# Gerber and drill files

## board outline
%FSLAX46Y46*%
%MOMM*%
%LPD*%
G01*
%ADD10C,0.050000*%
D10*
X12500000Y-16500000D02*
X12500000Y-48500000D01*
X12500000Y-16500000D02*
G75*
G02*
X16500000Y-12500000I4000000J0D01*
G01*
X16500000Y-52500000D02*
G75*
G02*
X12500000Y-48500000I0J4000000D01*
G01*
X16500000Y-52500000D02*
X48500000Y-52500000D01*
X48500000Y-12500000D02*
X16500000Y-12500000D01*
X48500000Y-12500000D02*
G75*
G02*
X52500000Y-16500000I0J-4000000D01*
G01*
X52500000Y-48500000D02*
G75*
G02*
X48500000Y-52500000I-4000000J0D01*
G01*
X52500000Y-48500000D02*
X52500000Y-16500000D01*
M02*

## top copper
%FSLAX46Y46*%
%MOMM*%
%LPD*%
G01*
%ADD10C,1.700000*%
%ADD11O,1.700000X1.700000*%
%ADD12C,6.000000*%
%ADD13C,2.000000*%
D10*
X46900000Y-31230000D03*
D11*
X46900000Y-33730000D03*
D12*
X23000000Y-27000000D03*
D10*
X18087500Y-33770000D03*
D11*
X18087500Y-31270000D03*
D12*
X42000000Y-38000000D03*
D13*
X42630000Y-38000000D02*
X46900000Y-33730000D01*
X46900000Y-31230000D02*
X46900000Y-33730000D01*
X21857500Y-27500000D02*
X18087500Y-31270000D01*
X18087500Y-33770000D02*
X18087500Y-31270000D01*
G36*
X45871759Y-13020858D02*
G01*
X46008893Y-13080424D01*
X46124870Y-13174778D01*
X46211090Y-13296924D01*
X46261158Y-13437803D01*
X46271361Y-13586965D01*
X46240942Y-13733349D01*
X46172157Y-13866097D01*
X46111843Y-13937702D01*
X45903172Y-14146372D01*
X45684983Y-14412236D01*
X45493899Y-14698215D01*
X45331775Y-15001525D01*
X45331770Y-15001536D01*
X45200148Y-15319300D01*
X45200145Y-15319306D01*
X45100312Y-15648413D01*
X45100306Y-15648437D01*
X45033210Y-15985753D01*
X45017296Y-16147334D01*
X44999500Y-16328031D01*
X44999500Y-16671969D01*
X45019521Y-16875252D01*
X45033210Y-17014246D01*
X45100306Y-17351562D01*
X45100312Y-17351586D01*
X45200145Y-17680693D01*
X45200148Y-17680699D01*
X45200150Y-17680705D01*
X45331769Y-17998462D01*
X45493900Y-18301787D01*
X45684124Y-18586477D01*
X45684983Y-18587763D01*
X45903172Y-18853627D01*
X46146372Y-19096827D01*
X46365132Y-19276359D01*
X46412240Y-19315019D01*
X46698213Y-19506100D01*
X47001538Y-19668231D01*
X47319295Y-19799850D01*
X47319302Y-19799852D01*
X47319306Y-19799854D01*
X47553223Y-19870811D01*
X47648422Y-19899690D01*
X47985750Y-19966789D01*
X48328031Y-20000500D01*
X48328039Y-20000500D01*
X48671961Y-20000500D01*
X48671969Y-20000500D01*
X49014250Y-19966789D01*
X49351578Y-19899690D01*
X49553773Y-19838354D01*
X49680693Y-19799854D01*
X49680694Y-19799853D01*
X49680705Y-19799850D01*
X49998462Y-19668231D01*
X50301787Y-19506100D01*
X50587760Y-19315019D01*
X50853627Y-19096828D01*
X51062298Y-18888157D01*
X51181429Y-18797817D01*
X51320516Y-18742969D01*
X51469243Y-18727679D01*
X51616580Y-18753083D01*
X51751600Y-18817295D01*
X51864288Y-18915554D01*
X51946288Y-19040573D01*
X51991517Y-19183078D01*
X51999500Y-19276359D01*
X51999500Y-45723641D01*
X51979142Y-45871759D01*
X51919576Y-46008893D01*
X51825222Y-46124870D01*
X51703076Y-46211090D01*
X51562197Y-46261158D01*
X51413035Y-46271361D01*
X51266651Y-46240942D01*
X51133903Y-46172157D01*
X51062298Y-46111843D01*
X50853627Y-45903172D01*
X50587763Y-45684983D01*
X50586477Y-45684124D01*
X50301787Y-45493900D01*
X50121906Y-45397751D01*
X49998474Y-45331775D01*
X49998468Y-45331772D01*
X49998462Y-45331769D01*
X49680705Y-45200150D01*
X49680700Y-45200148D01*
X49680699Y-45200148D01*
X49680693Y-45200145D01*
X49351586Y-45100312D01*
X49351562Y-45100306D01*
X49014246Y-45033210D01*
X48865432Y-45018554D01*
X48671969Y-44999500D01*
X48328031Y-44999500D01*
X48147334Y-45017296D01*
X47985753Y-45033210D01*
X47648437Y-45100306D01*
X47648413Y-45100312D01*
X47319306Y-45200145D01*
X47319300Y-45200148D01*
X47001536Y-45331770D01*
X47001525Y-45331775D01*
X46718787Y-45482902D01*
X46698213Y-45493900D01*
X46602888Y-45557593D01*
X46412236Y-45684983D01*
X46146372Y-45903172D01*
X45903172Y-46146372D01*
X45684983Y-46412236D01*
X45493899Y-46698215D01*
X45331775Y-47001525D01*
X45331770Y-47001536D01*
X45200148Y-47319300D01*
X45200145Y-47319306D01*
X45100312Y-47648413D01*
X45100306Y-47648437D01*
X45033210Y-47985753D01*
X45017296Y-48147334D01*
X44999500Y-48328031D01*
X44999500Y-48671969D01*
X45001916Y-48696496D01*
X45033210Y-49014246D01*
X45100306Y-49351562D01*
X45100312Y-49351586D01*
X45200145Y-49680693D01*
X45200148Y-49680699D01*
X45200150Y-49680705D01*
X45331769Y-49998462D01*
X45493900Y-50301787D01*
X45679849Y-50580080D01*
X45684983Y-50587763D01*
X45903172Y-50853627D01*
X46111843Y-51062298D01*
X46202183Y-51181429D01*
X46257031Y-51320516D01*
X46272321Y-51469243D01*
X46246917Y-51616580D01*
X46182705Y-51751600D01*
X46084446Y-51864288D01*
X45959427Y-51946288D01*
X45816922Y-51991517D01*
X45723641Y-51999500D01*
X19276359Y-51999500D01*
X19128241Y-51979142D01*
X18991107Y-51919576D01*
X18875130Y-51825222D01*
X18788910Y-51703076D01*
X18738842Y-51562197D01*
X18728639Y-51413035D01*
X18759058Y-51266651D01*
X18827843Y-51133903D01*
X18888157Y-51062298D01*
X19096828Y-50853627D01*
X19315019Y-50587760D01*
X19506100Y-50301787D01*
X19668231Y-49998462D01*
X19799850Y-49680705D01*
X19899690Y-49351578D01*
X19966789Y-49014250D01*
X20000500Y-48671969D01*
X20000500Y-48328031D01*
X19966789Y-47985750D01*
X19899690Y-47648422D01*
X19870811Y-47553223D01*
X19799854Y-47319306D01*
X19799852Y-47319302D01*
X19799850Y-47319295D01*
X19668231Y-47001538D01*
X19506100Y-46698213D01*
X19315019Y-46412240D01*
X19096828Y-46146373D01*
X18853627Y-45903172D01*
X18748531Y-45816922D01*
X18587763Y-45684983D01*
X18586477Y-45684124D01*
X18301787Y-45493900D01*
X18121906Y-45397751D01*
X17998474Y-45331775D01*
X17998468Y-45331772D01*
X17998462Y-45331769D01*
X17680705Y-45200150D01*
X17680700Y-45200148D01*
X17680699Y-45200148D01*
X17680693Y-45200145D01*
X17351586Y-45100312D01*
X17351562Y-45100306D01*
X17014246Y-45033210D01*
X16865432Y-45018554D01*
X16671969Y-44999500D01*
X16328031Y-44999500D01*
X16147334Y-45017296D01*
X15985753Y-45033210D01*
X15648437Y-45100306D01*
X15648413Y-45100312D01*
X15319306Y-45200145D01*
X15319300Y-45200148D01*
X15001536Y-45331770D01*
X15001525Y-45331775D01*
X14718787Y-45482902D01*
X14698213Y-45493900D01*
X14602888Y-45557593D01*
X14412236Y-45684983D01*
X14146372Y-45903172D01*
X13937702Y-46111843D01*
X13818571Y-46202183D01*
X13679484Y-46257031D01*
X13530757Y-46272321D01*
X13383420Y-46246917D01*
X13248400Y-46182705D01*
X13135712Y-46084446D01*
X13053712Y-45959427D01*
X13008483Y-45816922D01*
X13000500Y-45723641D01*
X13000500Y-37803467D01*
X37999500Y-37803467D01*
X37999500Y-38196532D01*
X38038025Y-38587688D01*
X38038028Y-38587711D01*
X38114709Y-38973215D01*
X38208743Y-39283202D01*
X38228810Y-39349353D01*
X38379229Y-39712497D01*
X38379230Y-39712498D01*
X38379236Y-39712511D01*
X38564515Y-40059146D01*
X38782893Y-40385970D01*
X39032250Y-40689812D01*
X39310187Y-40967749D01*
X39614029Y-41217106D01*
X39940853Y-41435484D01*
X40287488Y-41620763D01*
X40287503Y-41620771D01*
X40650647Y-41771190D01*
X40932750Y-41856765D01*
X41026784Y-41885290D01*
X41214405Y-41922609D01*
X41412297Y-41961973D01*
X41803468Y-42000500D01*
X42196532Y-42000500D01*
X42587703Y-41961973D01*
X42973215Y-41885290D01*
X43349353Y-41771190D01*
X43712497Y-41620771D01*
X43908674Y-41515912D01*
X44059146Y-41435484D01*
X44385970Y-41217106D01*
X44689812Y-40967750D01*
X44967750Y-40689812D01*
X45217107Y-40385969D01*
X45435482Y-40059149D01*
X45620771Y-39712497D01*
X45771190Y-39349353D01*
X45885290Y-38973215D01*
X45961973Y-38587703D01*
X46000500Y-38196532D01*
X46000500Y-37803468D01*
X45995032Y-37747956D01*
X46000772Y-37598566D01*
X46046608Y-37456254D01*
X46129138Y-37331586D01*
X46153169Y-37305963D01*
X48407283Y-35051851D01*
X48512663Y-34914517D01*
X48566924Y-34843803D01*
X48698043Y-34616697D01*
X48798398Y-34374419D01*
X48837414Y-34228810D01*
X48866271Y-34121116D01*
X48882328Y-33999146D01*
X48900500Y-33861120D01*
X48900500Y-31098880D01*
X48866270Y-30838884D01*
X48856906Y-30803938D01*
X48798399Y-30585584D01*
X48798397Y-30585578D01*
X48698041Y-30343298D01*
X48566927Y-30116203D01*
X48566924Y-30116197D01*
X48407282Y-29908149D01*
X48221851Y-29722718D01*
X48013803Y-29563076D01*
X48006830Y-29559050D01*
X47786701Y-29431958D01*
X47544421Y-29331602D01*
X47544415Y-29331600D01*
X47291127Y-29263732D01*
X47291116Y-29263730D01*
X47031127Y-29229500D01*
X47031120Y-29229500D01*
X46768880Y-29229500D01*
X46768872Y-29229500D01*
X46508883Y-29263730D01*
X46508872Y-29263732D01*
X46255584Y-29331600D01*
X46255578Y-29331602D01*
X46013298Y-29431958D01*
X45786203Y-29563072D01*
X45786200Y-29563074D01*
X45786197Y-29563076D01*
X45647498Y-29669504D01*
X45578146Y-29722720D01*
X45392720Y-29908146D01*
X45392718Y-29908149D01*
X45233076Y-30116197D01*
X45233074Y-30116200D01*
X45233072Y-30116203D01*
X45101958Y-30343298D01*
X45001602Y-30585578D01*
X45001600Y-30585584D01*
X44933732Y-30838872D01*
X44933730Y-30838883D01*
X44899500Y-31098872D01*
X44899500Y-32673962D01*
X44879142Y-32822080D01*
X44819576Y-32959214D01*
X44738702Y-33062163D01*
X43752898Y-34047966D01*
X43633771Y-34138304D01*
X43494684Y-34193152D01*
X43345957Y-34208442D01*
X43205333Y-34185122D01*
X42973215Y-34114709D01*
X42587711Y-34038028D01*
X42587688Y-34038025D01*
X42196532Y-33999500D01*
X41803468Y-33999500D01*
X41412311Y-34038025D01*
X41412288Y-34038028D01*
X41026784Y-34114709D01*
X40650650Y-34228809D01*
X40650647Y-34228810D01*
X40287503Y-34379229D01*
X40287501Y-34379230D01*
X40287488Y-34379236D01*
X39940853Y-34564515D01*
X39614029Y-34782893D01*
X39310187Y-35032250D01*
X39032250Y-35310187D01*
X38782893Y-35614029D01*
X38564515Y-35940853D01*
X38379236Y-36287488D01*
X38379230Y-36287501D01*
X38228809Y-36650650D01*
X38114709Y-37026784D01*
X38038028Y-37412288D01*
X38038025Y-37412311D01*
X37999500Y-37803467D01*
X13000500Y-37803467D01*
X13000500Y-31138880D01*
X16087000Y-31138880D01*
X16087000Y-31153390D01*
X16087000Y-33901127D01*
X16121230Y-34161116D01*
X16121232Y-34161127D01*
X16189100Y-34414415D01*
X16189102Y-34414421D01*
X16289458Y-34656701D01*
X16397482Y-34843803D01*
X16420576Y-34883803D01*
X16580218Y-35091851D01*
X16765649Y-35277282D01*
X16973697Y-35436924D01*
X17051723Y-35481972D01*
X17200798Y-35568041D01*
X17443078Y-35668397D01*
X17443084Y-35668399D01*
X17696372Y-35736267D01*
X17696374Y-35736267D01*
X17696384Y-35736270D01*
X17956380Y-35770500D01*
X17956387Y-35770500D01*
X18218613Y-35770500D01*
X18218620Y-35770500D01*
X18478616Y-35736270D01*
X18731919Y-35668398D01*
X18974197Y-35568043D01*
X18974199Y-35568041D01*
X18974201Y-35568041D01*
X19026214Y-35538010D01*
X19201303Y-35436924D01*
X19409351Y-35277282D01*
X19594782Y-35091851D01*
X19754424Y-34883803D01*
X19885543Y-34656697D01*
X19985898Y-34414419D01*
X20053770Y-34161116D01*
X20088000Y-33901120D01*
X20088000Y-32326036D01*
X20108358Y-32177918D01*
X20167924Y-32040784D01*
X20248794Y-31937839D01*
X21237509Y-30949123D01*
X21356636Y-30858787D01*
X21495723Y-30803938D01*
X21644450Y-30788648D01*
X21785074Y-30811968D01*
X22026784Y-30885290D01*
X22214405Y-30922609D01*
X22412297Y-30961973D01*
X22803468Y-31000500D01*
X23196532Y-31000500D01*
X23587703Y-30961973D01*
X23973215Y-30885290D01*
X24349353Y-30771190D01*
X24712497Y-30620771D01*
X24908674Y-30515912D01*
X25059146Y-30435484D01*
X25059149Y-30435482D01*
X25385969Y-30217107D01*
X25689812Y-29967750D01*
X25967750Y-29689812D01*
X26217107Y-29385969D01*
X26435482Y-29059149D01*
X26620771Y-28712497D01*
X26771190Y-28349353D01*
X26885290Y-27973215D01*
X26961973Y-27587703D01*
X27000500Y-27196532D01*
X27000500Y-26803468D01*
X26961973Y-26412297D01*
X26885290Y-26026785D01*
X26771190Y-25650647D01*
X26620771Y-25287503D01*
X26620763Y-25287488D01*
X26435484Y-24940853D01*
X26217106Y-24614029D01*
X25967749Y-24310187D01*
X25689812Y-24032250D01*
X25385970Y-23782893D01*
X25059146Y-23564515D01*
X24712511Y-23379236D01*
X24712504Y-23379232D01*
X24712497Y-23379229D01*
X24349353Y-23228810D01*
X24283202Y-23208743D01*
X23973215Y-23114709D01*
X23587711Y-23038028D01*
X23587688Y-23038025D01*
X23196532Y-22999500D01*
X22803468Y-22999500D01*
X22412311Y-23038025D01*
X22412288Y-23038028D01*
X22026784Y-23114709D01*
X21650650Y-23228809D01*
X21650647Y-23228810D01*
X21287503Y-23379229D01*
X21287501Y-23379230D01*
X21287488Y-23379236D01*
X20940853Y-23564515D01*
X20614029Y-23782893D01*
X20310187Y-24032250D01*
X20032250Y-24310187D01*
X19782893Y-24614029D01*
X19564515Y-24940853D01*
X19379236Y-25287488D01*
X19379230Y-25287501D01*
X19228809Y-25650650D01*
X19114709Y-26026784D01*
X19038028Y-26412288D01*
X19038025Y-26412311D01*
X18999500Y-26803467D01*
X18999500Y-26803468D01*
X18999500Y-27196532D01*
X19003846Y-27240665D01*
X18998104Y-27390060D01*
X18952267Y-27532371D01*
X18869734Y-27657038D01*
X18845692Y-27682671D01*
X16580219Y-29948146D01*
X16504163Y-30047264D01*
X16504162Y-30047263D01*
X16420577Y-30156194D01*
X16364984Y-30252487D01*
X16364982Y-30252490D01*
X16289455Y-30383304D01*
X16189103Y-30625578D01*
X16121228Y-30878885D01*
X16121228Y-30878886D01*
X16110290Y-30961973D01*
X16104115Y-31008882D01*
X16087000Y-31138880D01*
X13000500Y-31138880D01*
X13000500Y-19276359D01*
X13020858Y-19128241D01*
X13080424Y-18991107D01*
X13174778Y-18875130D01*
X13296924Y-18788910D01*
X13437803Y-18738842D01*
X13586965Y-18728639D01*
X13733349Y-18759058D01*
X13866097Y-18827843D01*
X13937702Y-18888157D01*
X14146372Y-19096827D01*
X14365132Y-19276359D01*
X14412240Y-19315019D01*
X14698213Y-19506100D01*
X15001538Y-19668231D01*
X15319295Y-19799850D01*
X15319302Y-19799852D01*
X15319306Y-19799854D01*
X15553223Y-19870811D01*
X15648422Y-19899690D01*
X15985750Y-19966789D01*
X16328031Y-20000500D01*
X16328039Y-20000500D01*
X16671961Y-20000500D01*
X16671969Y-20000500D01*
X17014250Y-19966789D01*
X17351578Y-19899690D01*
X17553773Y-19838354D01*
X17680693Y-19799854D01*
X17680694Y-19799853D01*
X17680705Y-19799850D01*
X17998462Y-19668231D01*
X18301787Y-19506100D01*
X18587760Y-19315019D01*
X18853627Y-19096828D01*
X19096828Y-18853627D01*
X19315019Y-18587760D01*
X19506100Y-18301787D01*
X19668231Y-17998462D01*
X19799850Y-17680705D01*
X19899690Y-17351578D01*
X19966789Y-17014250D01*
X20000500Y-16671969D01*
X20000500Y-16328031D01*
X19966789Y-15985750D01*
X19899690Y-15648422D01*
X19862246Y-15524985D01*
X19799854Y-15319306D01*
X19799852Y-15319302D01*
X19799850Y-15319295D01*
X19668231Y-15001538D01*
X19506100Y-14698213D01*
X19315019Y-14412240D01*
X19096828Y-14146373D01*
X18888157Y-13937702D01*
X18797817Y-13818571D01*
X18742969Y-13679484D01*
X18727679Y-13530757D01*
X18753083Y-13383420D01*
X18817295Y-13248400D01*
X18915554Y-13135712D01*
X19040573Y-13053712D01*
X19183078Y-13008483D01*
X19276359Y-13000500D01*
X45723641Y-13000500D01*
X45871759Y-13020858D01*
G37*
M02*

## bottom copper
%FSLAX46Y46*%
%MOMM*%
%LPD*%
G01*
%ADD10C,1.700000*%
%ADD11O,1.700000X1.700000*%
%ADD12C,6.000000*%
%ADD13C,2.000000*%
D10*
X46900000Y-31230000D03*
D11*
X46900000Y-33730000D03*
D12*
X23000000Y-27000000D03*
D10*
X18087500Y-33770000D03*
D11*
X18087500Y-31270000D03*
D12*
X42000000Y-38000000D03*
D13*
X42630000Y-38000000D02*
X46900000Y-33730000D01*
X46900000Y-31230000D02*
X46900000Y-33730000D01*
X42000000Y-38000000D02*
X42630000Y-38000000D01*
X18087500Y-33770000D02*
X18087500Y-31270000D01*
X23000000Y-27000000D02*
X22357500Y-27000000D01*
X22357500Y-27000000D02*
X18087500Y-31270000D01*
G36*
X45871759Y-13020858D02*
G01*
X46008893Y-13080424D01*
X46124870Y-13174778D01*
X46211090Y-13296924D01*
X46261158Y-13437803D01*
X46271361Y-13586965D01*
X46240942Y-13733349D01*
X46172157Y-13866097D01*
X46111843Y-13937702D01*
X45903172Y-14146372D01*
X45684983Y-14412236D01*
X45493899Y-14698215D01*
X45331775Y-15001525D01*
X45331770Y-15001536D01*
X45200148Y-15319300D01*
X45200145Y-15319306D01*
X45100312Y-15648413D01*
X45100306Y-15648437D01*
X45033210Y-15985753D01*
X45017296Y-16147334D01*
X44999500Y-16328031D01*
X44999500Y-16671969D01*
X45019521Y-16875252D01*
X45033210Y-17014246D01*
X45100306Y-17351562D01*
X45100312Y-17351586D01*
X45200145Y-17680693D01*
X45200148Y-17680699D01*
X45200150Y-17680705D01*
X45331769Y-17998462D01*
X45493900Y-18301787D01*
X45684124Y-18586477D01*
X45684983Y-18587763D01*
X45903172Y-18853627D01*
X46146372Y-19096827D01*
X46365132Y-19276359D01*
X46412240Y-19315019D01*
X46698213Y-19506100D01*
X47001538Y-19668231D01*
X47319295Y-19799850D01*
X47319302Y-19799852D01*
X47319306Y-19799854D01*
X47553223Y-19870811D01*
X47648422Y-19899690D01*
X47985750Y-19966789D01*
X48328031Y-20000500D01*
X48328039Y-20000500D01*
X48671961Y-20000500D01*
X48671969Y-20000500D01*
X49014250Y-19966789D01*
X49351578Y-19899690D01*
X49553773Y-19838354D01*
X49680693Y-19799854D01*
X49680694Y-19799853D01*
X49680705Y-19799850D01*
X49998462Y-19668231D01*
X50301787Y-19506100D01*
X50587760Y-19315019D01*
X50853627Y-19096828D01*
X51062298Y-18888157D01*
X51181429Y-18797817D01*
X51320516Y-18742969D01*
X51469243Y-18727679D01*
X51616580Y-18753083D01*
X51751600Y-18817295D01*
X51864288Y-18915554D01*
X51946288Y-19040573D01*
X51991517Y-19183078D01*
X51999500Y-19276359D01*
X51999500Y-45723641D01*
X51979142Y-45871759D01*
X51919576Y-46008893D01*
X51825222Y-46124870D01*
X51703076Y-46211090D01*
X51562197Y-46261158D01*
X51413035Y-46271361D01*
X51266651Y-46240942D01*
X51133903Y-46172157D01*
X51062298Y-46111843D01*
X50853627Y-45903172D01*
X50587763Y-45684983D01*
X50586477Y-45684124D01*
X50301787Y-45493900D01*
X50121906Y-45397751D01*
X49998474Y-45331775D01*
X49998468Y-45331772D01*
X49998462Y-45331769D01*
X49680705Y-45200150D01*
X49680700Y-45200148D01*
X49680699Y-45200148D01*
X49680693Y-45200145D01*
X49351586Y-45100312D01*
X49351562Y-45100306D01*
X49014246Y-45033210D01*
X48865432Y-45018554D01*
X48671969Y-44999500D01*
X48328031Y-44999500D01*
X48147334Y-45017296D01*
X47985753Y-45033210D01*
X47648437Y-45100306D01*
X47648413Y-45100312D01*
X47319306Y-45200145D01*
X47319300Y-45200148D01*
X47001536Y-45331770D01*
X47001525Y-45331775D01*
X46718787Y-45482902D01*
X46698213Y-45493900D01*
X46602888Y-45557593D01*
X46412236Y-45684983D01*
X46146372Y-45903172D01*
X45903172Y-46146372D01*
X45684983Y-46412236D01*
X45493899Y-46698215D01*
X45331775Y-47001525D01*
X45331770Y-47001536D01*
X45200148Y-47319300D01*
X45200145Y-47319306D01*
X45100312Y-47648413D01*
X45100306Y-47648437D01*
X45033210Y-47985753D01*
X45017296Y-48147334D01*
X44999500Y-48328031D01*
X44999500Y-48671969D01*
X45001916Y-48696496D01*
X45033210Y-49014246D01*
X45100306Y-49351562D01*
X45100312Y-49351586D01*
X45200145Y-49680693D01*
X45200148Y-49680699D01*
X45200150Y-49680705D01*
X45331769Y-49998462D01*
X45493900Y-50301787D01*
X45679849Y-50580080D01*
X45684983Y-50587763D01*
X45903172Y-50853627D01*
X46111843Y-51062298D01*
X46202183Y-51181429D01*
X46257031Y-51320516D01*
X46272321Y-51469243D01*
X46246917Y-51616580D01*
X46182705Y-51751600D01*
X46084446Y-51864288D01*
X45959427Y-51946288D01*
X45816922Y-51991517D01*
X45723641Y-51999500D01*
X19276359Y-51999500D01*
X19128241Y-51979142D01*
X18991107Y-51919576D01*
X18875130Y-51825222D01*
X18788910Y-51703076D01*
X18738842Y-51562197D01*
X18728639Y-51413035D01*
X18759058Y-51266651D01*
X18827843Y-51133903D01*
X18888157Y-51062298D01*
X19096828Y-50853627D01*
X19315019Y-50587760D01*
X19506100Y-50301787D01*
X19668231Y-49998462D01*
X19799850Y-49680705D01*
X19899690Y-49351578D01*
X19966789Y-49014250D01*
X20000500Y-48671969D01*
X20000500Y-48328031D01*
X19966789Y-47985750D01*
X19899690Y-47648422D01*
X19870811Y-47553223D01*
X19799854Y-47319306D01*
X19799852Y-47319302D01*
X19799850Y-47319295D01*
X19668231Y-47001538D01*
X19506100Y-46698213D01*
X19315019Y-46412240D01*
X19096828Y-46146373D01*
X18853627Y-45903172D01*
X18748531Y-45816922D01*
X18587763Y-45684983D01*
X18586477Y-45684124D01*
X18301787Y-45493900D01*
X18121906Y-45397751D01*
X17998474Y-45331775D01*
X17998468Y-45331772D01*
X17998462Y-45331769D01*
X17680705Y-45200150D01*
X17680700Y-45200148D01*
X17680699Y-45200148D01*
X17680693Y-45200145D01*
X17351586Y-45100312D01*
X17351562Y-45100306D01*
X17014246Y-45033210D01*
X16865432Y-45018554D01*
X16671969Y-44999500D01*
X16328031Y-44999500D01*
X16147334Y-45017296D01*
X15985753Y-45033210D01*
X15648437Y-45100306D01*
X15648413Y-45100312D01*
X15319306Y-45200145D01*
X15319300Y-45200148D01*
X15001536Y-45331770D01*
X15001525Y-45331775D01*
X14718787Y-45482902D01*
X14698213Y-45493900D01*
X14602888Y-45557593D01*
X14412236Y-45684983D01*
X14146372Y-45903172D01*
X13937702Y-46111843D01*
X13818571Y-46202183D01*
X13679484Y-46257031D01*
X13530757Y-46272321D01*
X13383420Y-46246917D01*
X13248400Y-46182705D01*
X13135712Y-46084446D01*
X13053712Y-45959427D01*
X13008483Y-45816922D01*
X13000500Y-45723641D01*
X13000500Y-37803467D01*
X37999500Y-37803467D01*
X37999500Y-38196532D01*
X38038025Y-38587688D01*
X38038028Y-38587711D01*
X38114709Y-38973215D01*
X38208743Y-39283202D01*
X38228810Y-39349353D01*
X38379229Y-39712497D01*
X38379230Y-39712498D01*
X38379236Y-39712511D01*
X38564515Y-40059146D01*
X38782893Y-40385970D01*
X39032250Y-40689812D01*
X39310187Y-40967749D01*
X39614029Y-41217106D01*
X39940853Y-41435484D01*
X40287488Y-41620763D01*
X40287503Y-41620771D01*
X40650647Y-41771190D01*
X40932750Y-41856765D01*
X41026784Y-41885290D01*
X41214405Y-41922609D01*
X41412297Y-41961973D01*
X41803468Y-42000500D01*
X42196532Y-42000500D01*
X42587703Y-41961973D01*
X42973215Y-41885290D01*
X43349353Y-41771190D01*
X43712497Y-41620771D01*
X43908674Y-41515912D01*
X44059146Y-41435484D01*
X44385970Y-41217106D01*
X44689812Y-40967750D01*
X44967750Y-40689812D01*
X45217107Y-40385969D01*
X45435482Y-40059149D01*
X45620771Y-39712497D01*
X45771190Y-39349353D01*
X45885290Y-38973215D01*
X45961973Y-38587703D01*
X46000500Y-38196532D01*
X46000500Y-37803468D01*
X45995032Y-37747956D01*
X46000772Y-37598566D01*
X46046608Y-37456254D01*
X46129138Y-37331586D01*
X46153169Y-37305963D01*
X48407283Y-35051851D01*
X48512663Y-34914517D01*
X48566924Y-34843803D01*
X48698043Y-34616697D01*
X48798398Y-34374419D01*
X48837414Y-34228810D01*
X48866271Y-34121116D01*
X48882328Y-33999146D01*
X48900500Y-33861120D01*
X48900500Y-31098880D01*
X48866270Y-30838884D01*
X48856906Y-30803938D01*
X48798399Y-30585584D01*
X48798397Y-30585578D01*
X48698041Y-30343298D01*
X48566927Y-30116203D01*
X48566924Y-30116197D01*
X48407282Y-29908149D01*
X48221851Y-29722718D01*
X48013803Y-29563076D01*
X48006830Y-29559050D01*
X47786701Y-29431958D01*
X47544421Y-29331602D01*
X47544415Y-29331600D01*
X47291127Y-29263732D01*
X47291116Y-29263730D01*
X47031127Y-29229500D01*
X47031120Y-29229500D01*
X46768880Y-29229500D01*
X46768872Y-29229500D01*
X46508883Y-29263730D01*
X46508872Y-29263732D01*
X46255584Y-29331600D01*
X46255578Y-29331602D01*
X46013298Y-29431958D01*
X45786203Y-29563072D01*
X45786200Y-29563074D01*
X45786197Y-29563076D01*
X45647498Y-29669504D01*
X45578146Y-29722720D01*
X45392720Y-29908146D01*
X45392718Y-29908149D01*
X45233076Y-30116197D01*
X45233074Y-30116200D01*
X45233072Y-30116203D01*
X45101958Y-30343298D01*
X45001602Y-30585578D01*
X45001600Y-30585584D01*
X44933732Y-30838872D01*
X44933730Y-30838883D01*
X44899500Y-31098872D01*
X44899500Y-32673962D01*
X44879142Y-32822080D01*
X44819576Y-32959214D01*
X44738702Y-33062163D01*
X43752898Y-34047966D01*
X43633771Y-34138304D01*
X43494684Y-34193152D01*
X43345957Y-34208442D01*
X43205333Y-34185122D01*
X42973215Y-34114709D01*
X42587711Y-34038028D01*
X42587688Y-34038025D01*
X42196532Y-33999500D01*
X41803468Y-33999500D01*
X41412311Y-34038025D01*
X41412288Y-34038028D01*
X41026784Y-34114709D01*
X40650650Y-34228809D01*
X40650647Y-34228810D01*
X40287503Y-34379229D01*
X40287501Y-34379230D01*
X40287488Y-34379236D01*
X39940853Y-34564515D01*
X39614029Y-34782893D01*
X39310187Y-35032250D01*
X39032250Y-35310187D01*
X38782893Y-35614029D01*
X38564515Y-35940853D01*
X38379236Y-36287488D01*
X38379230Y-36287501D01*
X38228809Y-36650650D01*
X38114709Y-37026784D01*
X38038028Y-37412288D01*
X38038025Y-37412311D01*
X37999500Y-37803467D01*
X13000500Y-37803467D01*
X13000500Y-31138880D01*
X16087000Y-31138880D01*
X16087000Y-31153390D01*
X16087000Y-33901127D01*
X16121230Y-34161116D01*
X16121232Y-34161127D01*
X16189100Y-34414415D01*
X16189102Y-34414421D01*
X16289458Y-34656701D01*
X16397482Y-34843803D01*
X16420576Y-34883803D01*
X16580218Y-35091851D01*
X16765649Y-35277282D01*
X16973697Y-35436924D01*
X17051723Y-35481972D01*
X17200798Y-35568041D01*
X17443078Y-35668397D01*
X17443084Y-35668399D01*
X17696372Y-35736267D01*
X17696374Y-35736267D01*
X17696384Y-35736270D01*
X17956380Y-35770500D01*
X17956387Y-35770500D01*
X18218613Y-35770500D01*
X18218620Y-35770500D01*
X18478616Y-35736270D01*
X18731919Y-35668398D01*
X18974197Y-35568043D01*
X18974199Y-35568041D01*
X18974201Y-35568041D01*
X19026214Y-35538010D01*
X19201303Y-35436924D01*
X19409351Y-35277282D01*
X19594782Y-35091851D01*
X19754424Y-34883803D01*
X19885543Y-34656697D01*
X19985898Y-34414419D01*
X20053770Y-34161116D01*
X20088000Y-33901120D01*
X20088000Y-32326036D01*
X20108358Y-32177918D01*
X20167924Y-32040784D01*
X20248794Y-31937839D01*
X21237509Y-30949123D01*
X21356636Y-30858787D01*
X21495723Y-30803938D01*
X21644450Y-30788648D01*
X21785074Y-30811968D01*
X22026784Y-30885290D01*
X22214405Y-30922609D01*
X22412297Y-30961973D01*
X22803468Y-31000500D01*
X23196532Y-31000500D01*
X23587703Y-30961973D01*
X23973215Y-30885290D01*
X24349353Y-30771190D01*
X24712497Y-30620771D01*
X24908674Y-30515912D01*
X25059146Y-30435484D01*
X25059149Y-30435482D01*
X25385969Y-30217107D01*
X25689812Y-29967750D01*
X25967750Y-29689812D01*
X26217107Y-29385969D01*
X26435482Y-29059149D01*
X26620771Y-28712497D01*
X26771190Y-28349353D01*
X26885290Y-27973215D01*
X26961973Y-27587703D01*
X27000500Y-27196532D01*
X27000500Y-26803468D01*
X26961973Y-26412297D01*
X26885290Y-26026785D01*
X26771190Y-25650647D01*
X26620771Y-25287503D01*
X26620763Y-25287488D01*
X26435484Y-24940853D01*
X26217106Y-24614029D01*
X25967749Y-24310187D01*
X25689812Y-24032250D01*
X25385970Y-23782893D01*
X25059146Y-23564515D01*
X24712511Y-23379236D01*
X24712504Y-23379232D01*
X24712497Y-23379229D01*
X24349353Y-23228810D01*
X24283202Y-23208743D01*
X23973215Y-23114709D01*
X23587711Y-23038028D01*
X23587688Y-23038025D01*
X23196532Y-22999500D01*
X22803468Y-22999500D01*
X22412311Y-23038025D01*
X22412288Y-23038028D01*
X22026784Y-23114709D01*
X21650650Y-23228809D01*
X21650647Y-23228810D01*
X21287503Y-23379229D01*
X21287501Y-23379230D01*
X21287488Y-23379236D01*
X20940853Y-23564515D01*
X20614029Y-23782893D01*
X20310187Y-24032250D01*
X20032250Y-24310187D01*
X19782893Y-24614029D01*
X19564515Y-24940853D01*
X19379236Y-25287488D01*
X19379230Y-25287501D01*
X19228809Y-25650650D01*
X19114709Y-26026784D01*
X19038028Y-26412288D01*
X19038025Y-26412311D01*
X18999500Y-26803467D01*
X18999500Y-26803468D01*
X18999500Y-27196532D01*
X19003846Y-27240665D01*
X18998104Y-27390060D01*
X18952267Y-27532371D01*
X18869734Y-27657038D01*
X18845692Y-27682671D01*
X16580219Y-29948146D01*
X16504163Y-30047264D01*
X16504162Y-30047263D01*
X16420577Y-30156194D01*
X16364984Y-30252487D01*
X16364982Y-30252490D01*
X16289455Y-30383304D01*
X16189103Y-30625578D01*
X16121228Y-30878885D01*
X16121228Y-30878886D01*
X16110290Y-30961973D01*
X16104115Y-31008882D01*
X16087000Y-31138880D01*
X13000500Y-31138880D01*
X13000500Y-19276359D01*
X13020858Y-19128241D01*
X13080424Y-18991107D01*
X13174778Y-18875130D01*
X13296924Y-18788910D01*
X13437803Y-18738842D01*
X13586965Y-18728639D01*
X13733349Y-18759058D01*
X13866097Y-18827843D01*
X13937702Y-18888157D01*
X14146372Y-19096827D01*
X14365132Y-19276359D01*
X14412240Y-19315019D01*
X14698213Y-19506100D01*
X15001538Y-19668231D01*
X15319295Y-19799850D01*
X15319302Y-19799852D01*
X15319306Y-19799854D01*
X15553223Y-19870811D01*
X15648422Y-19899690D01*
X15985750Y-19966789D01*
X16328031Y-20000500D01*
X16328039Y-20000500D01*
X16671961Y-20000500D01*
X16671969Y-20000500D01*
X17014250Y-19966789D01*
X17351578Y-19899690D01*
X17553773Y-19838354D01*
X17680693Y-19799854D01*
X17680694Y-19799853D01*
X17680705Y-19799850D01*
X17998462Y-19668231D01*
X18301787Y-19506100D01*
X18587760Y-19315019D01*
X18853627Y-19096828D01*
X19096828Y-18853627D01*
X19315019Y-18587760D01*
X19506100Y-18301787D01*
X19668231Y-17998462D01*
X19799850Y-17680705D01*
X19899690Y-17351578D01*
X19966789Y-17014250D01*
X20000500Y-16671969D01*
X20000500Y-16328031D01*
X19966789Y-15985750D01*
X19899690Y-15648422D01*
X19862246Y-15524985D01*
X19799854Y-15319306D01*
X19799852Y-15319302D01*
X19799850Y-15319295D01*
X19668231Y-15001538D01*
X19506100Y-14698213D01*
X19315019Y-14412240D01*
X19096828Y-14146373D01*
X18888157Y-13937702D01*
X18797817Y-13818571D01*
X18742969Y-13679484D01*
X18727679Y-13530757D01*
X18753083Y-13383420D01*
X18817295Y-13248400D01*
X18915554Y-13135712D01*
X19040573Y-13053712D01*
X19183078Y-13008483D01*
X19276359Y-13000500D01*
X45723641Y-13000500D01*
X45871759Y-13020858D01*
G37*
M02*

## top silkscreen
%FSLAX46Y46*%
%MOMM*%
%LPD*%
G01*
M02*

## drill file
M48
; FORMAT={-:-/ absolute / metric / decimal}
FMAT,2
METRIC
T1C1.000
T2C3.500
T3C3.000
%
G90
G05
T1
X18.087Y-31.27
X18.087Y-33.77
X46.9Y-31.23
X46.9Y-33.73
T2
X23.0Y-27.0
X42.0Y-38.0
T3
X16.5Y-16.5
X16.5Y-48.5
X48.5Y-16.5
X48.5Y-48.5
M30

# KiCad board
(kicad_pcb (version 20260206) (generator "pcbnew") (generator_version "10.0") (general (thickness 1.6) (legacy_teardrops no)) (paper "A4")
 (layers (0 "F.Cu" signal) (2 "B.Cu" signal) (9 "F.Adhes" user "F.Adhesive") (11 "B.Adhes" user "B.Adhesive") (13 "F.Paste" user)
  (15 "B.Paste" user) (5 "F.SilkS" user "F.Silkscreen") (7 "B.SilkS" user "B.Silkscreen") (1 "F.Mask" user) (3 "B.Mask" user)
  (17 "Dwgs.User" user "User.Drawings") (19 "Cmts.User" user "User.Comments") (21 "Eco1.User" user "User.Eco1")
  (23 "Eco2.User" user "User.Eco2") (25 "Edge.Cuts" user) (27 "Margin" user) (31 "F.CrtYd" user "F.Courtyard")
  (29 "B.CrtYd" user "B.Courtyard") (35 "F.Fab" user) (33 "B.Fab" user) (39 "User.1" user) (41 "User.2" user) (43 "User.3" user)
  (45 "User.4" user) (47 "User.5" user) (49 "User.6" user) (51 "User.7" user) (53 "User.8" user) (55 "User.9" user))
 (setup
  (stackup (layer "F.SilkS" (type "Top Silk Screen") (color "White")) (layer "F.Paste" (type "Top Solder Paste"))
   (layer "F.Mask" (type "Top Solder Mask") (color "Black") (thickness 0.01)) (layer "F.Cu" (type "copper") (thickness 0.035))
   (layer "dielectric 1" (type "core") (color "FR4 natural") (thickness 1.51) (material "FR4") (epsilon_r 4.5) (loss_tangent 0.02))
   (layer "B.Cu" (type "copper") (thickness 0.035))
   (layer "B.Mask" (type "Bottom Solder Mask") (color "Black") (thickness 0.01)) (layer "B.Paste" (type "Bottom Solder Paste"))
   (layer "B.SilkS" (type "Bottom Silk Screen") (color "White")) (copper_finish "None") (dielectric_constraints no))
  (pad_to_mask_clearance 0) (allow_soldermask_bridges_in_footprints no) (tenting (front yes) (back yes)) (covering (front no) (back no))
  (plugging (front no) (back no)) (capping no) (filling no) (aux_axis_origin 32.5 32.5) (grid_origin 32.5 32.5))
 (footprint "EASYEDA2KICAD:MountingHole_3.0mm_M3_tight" (layer "F.Cu") (at 48.5 48.5 -90)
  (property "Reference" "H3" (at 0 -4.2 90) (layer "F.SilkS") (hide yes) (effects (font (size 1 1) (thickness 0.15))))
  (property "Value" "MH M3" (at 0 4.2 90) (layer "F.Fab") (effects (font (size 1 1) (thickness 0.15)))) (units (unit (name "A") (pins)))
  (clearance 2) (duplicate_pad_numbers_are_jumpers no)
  (pad "" np_thru_hole circle (at 0 0 270) (size 3 3) (drill 3) (layers "*.Cu" "*.Mask")))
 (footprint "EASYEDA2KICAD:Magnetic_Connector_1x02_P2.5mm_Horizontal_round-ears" (layer "F.Cu") (at 47 32.5)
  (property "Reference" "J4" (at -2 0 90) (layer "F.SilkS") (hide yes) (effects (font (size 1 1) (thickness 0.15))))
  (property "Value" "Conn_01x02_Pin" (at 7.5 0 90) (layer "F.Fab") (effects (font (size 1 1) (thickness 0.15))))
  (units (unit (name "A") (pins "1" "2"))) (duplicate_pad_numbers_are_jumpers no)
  (pad "1" thru_hole circle (at -0.1 -1.27) (size 1.7 1.7) (drill 1) (layers "*.Cu" "*.Mask") (remove_unused_layers no)
   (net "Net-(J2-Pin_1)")
   (teardrops (best_length_ratio 0.5) (max_length 1) (best_width_ratio 1) (max_width 2) (curved_edges yes) (filter_ratio 0.9) (enabled yes)
    (allow_two_segments yes) (prefer_zone_connections yes)))
  (pad "2" thru_hole oval (at -0.1 1.23) (size 1.7 1.7) (drill 1) (layers "*.Cu" "*.Mask") (remove_unused_layers no) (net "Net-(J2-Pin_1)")
   (teardrops (best_length_ratio 0.5) (max_length 1) (best_width_ratio 1) (max_width 2) (curved_edges yes) (filter_ratio 0.9) (enabled yes)
    (allow_two_segments yes) (prefer_zone_connections yes))))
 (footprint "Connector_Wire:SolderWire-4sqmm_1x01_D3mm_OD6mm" (layer "F.Cu") (at 23 27 -90)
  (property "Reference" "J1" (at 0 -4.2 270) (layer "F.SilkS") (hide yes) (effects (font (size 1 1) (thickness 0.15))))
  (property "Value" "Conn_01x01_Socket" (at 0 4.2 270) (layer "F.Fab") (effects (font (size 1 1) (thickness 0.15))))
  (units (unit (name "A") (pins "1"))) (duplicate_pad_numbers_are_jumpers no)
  (pad "1" thru_hole circle (at 0 0 270) (size 6 6) (drill 3.5) (layers "*.Cu" "*.Mask") (remove_unused_layers no) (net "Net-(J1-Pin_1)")
   (teardrops (best_length_ratio 0.5) (max_length 1) (best_width_ratio 1) (max_width 2) (curved_edges yes) (filter_ratio 0.9) (enabled yes)
    (allow_two_segments yes) (prefer_zone_connections yes))))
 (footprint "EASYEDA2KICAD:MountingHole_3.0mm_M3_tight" (layer "F.Cu") (at 48.5 16.5 -90)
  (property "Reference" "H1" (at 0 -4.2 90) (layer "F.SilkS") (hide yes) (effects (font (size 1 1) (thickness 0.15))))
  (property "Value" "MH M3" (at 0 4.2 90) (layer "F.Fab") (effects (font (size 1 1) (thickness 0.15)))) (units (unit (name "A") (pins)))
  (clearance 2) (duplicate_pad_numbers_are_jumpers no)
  (pad "" np_thru_hole circle (at 0 0 270) (size 3 3) (drill 3) (layers "*.Cu" "*.Mask")))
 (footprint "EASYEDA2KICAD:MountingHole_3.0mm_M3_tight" (layer "F.Cu") (at 16.5 48.5 -90)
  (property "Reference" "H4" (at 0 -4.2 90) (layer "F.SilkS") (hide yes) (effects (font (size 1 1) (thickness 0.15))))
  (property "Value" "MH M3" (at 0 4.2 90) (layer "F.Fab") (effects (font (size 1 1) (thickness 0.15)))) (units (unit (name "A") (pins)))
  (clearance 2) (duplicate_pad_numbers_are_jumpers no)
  (pad "" np_thru_hole circle (at 0 0 270) (size 3 3) (drill 3) (layers "*.Cu" "*.Mask")))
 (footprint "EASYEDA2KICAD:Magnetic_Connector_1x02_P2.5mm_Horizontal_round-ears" (layer "F.Cu") (at 17.9875 32.5 180)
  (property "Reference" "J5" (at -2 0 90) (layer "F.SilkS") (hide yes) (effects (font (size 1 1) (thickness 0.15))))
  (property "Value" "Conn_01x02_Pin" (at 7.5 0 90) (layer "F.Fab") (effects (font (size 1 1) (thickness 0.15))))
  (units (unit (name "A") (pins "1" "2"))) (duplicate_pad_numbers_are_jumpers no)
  (pad "1" thru_hole circle (at -0.1 -1.27 180) (size 1.7 1.7) (drill 1) (layers "*.Cu" "*.Mask") (remove_unused_layers no)
   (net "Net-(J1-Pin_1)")
   (teardrops (best_length_ratio 0.5) (max_length 1) (best_width_ratio 1) (max_width 2) (curved_edges yes) (filter_ratio 0.9) (enabled yes)
    (allow_two_segments yes) (prefer_zone_connections yes)))
  (pad "2" thru_hole oval (at -0.1 1.23 180) (size 1.7 1.7) (drill 1) (layers "*.Cu" "*.Mask") (remove_unused_layers no)
   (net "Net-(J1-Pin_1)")
   (teardrops (best_length_ratio 0.5) (max_length 1) (best_width_ratio 1) (max_width 2) (curved_edges yes) (filter_ratio 0.9) (enabled yes)
    (allow_two_segments yes) (prefer_zone_connections yes))))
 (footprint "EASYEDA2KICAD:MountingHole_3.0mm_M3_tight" (layer "F.Cu") (at 16.5 16.5 -90)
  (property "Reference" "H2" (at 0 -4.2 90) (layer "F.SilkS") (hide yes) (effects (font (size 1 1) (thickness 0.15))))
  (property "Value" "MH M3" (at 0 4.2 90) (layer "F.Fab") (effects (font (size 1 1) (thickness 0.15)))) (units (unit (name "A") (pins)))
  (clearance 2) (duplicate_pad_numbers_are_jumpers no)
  (pad "" np_thru_hole circle (at 0 0 270) (size 3 3) (drill 3) (layers "*.Cu" "*.Mask")))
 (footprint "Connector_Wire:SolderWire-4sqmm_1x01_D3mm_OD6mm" (layer "F.Cu") (at 42 38 -90)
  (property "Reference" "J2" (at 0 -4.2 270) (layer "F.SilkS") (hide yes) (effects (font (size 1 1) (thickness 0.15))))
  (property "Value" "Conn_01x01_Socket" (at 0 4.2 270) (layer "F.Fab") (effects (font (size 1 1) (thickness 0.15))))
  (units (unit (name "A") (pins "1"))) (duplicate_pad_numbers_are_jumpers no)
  (pad "1" thru_hole circle (at 0 0 270) (size 6 6) (drill 3.5) (layers "*.Cu" "*.Mask") (remove_unused_layers no) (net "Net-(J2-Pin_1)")
   (teardrops (best_length_ratio 0.5) (max_length 1) (best_width_ratio 1) (max_width 2) (curved_edges yes) (filter_ratio 0.9) (enabled yes)
    (allow_two_segments yes) (prefer_zone_connections yes))))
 (gr_line (start 12.5 16.5) (end 12.5 48.5) (stroke (width 0.05) (type default)) (layer "Edge.Cuts"))
 (gr_arc (start 12.5 16.5) (mid 13.671573 13.671573) (end 16.5 12.5) (stroke (width 0.05) (type default)) (layer "Edge.Cuts"))
 (gr_arc (start 16.5 52.5) (mid 13.671573 51.328427) (end 12.5 48.5) (stroke (width 0.05) (type default)) (layer "Edge.Cuts"))
 (gr_line (start 16.5 52.5) (end 48.5 52.5) (stroke (width 0.05) (type default)) (layer "Edge.Cuts"))
 (gr_line (start 48.5 12.5) (end 16.5 12.5) (stroke (width 0.05) (type default)) (layer "Edge.Cuts"))
 (gr_arc (start 48.5 12.5) (mid 51.328427 13.671573) (end 52.5 16.5) (stroke (width 0.05) (type default)) (layer "Edge.Cuts"))
 (gr_arc (start 52.5 48.5) (mid 51.328427 51.328427) (end 48.5 52.5) (stroke (width 0.05) (type default)) (layer "Edge.Cuts"))
 (gr_line (start 52.5 48.5) (end 52.5 16.5) (stroke (width 0.05) (type default)) (layer "Edge.Cuts"))
 (segment (start 42.63 38) (end 46.9 33.73) (width 2) (layer "F.Cu") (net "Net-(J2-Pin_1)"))
 (segment (start 46.9 31.23) (end 46.9 33.73) (width 2) (layer "F.Cu") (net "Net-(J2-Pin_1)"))
 (segment (start 42.63 38) (end 46.9 33.73) (width 2) (layer "B.Cu") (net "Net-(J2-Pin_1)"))
 (segment (start 46.9 31.23) (end 46.9 33.73) (width 2) (layer "B.Cu") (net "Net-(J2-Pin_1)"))
 (segment (start 42 38) (end 42.63 38) (width 2) (layer "B.Cu") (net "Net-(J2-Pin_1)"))
 (segment (start 21.8575 27.5) (end 18.0875 31.27) (width 2) (layer "F.Cu") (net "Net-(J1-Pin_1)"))
 (segment (start 18.0875 33.77) (end 18.0875 31.27) (width 2) (layer "F.Cu") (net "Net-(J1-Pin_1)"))
 (segment (start 18.0875 33.77) (end 18.0875 31.27) (width 2) (layer "B.Cu") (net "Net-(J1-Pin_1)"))
 (segment (start 23 27) (end 22.3575 27) (width 2) (layer "B.Cu") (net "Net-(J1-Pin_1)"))
 (segment (start 22.3575 27) (end 18.0875 31.27) (width 2) (layer "B.Cu") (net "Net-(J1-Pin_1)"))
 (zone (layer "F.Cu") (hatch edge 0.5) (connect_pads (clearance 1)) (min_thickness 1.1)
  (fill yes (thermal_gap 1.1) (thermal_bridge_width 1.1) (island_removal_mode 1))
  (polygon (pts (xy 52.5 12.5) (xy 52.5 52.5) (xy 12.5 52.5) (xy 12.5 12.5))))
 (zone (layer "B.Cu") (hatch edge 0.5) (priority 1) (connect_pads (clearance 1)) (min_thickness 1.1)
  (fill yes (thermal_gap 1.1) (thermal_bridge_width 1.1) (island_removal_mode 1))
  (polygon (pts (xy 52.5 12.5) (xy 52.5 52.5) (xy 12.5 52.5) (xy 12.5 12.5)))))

